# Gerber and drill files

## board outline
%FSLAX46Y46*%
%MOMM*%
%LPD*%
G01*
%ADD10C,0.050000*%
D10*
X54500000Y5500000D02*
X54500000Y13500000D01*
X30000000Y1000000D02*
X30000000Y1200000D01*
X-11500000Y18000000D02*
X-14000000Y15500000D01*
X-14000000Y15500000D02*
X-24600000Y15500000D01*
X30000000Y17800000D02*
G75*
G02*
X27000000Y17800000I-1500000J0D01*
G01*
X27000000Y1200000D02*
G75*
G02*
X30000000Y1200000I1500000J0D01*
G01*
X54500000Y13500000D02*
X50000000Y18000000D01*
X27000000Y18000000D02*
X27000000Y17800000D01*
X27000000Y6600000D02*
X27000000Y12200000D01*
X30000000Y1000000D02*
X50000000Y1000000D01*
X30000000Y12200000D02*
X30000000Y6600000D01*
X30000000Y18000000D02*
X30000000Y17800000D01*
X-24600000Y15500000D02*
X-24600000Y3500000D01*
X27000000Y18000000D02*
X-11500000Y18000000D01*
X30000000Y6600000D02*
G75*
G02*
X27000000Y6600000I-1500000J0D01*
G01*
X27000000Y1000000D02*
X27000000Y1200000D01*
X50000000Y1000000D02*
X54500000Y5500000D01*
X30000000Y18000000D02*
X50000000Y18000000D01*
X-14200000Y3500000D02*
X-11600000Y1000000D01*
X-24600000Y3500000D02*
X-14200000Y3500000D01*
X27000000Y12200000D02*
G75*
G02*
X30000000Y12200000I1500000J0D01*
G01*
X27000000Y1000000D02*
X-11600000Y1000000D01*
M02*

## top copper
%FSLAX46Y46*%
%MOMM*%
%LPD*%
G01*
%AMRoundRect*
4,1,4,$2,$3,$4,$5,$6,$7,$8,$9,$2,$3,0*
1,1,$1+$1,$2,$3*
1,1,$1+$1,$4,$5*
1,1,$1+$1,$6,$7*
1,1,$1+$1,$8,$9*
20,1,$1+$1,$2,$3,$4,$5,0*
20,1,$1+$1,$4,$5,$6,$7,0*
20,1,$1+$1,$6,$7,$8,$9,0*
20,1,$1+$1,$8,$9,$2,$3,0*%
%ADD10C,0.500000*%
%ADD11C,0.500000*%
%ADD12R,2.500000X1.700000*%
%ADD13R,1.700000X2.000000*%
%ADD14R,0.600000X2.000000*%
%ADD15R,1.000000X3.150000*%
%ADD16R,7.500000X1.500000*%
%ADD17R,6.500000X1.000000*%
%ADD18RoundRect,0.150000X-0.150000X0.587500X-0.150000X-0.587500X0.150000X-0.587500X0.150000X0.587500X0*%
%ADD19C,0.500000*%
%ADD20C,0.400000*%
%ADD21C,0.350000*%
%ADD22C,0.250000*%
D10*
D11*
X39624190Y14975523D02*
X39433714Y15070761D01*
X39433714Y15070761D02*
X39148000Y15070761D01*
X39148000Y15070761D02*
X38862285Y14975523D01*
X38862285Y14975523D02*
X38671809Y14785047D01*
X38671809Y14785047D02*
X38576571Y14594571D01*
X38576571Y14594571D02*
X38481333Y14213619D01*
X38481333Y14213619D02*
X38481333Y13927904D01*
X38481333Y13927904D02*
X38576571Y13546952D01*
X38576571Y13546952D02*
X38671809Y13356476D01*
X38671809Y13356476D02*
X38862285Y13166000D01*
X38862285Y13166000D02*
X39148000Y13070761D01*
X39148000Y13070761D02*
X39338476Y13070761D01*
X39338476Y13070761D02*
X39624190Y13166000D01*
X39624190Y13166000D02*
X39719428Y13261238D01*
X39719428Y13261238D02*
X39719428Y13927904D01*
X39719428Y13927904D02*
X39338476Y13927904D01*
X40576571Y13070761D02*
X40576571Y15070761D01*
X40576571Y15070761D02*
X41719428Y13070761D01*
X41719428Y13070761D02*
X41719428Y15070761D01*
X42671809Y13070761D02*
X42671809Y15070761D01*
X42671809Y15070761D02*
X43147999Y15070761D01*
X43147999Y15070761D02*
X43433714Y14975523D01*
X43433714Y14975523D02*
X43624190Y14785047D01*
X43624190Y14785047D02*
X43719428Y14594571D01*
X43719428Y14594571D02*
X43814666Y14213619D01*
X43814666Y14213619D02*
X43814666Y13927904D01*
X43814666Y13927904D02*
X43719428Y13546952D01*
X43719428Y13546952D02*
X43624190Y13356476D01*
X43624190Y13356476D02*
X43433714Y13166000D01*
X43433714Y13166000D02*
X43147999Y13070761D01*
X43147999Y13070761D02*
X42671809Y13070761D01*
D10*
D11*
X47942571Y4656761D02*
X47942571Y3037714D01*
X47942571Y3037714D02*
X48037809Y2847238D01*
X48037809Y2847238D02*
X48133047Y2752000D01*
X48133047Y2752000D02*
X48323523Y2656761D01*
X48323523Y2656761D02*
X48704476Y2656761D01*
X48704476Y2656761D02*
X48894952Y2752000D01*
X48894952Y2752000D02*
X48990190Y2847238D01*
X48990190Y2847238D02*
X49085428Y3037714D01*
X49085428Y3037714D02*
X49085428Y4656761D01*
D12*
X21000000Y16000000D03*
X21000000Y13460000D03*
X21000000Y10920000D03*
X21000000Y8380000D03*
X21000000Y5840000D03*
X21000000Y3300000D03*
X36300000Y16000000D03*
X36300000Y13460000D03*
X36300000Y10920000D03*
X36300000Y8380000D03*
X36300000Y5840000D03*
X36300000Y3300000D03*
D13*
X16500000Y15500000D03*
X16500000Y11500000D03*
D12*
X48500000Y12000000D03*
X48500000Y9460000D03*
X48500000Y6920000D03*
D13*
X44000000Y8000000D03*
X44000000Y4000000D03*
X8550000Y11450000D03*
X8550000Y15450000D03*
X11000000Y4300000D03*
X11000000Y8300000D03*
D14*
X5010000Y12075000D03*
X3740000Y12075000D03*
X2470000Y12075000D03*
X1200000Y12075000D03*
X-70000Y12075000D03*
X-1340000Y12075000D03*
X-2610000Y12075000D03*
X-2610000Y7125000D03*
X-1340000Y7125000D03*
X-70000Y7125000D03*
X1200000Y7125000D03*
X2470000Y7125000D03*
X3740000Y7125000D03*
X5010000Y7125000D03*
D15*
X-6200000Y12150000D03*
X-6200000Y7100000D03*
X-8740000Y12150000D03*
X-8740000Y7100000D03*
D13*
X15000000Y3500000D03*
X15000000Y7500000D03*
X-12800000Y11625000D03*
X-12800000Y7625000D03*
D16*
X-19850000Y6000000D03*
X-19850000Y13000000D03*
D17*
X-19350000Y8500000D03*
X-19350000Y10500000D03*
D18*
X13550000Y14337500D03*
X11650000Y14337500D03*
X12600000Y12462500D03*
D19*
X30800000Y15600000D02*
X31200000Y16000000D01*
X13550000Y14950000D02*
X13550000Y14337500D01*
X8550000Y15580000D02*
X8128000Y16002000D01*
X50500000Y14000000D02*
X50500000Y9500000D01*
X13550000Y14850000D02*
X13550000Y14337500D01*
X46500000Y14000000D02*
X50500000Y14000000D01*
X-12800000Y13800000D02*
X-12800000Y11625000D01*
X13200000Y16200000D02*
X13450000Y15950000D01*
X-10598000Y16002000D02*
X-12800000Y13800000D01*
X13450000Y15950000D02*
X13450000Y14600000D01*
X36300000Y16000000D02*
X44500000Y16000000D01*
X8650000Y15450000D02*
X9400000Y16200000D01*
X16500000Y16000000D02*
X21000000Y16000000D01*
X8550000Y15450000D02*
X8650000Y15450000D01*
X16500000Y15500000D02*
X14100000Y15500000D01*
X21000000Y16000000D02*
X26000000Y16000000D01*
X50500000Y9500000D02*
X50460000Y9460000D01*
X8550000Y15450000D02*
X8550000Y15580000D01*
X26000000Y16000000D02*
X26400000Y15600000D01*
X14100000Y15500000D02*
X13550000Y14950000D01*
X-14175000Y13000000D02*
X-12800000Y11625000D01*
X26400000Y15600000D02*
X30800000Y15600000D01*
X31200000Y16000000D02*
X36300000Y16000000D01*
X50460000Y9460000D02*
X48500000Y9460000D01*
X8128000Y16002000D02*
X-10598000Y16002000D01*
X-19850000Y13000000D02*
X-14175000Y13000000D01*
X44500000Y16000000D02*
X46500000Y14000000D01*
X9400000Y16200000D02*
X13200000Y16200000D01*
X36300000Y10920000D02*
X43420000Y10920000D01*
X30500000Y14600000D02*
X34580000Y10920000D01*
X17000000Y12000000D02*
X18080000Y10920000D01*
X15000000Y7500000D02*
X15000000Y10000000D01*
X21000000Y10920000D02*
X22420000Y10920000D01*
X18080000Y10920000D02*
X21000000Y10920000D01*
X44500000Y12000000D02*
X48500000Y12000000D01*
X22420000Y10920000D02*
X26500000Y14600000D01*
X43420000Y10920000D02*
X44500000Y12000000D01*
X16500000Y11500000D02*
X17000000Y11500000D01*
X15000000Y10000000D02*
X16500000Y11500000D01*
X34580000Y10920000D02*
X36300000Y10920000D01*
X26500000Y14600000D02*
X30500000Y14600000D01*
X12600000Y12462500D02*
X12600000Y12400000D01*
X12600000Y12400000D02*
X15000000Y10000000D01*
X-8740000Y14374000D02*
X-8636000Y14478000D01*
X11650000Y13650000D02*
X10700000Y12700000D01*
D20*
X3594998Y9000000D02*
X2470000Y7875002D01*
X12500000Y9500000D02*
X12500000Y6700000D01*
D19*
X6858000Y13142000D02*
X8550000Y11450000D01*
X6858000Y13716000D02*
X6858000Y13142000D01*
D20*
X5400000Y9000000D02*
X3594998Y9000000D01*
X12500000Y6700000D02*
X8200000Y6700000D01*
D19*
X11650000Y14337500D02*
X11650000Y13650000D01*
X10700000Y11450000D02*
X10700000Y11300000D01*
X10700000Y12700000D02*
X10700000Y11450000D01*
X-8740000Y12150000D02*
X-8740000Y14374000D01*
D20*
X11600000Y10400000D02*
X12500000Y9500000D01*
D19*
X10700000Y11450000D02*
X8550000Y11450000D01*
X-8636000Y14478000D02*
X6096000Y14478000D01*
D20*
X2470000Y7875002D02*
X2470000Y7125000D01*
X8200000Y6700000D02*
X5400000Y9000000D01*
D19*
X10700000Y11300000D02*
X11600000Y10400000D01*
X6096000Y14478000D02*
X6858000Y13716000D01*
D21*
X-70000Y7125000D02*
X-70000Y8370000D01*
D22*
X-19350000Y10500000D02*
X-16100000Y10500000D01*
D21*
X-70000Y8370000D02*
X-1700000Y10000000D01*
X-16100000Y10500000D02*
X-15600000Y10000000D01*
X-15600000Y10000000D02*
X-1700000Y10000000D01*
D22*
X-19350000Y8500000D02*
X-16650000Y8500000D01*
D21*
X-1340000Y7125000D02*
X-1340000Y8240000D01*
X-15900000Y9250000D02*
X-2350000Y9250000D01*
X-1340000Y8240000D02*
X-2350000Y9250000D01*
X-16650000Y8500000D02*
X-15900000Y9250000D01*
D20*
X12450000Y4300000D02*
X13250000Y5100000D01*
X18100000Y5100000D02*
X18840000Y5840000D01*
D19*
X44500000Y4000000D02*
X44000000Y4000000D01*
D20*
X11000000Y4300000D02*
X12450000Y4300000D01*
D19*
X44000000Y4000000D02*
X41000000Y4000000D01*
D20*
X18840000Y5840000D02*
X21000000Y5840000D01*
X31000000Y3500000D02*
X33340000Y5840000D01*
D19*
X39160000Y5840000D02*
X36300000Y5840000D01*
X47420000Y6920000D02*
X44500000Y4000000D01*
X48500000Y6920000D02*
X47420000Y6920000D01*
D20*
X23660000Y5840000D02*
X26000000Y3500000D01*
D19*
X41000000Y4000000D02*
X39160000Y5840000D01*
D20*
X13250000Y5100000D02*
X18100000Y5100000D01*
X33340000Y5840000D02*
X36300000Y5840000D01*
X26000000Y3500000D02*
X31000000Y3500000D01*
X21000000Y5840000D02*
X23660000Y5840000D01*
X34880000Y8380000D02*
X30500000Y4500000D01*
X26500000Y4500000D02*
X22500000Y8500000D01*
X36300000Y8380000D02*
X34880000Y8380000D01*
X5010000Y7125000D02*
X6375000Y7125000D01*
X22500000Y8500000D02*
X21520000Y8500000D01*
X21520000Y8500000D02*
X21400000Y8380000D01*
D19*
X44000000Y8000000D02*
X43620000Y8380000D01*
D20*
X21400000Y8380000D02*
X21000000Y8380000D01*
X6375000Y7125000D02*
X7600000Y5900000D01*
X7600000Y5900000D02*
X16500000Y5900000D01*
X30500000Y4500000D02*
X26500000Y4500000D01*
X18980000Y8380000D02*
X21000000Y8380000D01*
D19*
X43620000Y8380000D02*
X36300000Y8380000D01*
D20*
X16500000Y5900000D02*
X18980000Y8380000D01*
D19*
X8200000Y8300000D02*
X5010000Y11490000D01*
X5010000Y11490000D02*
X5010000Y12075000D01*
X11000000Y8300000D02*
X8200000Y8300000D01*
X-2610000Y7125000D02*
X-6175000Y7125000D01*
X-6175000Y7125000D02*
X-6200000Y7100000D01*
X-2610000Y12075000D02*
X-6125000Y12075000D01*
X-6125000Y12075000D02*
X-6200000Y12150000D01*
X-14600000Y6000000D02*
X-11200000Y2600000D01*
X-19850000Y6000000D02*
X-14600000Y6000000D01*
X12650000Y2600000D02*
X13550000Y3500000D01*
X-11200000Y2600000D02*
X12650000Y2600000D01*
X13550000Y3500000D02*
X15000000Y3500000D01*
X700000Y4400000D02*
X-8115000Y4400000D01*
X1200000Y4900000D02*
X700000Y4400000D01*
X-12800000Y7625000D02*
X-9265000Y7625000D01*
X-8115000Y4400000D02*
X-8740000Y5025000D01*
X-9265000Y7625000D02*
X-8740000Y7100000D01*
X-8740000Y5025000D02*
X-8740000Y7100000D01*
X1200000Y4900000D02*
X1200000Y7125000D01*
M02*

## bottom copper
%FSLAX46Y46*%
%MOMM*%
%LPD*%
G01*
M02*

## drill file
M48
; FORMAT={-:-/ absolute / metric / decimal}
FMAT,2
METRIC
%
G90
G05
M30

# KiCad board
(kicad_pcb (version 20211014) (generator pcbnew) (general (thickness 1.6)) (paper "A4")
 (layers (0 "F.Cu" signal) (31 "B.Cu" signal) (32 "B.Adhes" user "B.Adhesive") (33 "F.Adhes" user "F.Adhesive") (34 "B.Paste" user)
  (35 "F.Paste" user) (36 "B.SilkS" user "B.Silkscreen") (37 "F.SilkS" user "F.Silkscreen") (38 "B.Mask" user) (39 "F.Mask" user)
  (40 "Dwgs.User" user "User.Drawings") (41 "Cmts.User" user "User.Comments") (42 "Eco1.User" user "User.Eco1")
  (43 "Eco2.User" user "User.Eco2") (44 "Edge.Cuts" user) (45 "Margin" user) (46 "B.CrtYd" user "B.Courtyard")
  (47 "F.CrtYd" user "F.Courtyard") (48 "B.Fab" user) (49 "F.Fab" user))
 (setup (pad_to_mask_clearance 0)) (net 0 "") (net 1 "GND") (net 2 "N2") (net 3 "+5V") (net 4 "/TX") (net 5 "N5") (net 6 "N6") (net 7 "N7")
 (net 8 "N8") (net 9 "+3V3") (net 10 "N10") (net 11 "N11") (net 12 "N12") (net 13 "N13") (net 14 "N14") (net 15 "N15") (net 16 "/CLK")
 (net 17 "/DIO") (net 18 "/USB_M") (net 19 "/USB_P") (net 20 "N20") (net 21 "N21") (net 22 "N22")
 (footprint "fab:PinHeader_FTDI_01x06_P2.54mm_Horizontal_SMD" (layer "F.Cu") (at 21 -16)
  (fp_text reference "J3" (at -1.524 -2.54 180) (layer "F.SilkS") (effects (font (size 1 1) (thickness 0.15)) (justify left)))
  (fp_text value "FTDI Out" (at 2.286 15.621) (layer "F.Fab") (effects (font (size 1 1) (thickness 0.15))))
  (pad "1" smd rect locked (at 0 0) (size 2.5 1.7) (layers "F.Cu" "F.Paste" "F.Mask") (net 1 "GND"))
  (pad "2" smd rect locked (at 0 2.54) (size 2.5 1.7) (layers "F.Cu" "F.Paste" "F.Mask") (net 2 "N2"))
  (pad "3" smd rect locked (at 0 5.08) (size 2.5 1.7) (layers "F.Cu" "F.Paste" "F.Mask") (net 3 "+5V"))
  (pad "4" smd rect locked (at 0 7.62) (size 2.5 1.7) (layers "F.Cu" "F.Paste" "F.Mask") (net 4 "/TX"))
  (pad "5" smd rect locked (at 0 10.16) (size 2.5 1.7) (layers "F.Cu" "F.Paste" "F.Mask") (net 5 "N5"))
  (pad "6" smd rect locked (at 0 12.7) (size 2.5 1.7) (layers "F.Cu" "F.Paste" "F.Mask") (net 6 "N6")))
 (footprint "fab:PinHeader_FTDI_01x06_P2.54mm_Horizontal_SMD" (layer "F.Cu") (at 36.3 -16)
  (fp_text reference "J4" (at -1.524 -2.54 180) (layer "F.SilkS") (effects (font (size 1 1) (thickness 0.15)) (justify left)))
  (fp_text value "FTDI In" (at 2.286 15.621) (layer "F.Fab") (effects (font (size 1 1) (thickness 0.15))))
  (pad "1" smd rect locked (at 0 0) (size 2.5 1.7) (layers "F.Cu" "F.Paste" "F.Mask") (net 1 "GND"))
  (pad "2" smd rect locked (at 0 2.54) (size 2.5 1.7) (layers "F.Cu" "F.Paste" "F.Mask") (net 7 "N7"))
  (pad "3" smd rect locked (at 0 5.08) (size 2.5 1.7) (layers "F.Cu" "F.Paste" "F.Mask") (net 3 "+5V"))
  (pad "4" smd rect locked (at 0 7.62) (size 2.5 1.7) (layers "F.Cu" "F.Paste" "F.Mask") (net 4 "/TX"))
  (pad "5" smd rect locked (at 0 10.16) (size 2.5 1.7) (layers "F.Cu" "F.Paste" "F.Mask") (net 5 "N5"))
  (pad "6" smd rect locked (at 0 12.7) (size 2.5 1.7) (layers "F.Cu" "F.Paste" "F.Mask") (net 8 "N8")))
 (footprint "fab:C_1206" (layer "F.Cu") (at 16.5 -13.5 -90)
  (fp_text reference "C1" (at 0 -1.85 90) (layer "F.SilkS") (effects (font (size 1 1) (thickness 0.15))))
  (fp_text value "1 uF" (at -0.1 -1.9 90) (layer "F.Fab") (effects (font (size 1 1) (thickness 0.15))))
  (pad "1" smd rect locked (at -2 0 270) (size 2 1.7) (layers "F.Cu" "F.Paste" "F.Mask") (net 1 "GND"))
  (pad "2" smd rect locked (at 2 0 270) (size 2 1.7) (layers "F.Cu" "F.Paste" "F.Mask") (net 3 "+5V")))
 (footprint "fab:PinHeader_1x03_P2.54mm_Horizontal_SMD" (layer "F.Cu") (at 48.5 -12)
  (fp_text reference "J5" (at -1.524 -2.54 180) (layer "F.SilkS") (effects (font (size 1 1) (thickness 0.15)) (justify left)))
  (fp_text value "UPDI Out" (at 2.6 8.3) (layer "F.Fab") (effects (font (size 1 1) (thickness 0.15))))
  (pad "1" smd rect locked (at 0 0) (size 2.5 1.7) (layers "F.Cu" "F.Paste" "F.Mask") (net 3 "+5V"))
  (pad "2" smd rect locked (at 0 2.54) (size 2.5 1.7) (layers "F.Cu" "F.Paste" "F.Mask") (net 1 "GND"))
  (pad "3" smd rect locked (at 0 5.08) (size 2.5 1.7) (layers "F.Cu" "F.Paste" "F.Mask") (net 5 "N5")))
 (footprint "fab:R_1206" (layer "F.Cu") (at 44 -6 -90)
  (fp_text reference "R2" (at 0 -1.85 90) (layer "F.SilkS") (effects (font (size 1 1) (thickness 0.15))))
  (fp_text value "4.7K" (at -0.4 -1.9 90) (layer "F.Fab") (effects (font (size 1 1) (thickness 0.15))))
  (pad "1" smd rect locked (at -2 0 270) (size 2 1.7) (layers "F.Cu" "F.Paste" "F.Mask") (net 4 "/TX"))
  (pad "2" smd rect locked (at 2 0 270) (size 2 1.7) (layers "F.Cu" "F.Paste" "F.Mask") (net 5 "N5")))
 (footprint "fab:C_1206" (layer "F.Cu") (at 8.55 -13.45 90)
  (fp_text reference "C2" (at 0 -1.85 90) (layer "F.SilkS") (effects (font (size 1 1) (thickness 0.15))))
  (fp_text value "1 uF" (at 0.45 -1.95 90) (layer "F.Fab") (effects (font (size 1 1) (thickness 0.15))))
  (pad "1" smd rect locked (at -2 0 90) (size 2 1.7) (layers "F.Cu" "F.Paste" "F.Mask") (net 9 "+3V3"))
  (pad "2" smd rect locked (at 2 0 90) (size 2 1.7) (layers "F.Cu" "F.Paste" "F.Mask") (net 1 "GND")))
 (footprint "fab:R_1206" (layer "F.Cu") (at 11 -6.3 90)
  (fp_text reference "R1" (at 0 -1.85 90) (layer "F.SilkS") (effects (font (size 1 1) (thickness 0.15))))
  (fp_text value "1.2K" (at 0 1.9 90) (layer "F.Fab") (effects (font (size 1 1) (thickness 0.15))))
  (pad "1" smd rect locked (at -2 0 90) (size 2 1.7) (layers "F.Cu" "F.Paste" "F.Mask") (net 5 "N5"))
  (pad "2" smd rect locked (at 2 0 90) (size 2 1.7) (layers "F.Cu" "F.Paste" "F.Mask") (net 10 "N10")))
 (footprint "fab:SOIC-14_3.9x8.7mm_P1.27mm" (layer "F.Cu") (at 1.2 -9.6 -90)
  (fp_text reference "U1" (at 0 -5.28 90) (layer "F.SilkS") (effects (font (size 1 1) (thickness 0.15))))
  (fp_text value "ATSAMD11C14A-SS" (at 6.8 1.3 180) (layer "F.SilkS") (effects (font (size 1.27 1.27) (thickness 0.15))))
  (pad "1" smd rect locked (at -2.475 -3.81 270) (size 2 0.6) (layers "F.Cu" "F.Paste" "F.Mask") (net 10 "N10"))
  (pad "2" smd rect locked (at -2.475 -2.54 270) (size 2 0.6) (layers "F.Cu" "F.Paste" "F.Mask") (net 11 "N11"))
  (pad "3" smd rect locked (at -2.475 -1.27 270) (size 2 0.6) (layers "F.Cu" "F.Paste" "F.Mask") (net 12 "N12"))
  (pad "4" smd rect locked (at -2.475 0 270) (size 2 0.6) (layers "F.Cu" "F.Paste" "F.Mask") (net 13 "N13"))
  (pad "5" smd rect locked (at -2.475 1.27 270) (size 2 0.6) (layers "F.Cu" "F.Paste" "F.Mask") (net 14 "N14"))
  (pad "6" smd rect locked (at -2.475 2.54 270) (size 2 0.6) (layers "F.Cu" "F.Paste" "F.Mask") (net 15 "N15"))
  (pad "7" smd rect locked (at -2.475 3.81 270) (size 2 0.6) (layers "F.Cu" "F.Paste" "F.Mask") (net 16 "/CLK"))
  (pad "8" smd rect locked (at 2.475 3.81 270) (size 2 0.6) (layers "F.Cu" "F.Paste" "F.Mask") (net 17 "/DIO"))
  (pad "9" smd rect locked (at 2.475 2.54 270) (size 2 0.6) (layers "F.Cu" "F.Paste" "F.Mask") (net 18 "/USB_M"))
  (pad "10" smd rect locked (at 2.475 1.27 270) (size 2 0.6) (layers "F.Cu" "F.Paste" "F.Mask") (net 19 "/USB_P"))
  (pad "11" smd rect locked (at 2.475 0 270) (size 2 0.6) (layers "F.Cu" "F.Paste" "F.Mask") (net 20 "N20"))
  (pad "12" smd rect locked (at 2.475 -1.27 270) (size 2 0.6) (layers "F.Cu" "F.Paste" "F.Mask") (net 9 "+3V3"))
  (pad "13" smd rect locked (at 2.475 -2.54 270) (size 2 0.6) (layers "F.Cu" "F.Paste" "F.Mask") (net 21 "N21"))
  (pad "14" smd rect locked (at 2.475 -3.81 270) (size 2 0.6) (layers "F.Cu" "F.Paste" "F.Mask") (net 4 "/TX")))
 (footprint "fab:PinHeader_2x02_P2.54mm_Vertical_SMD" (layer "F.Cu") (at -7.47 -9.625 -90)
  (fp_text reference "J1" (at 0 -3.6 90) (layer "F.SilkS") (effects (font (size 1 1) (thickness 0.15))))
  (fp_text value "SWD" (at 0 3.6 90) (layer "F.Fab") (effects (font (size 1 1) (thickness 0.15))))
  (pad "1" smd rect locked (at -2.525 -1.27 270) (size 3.15 1) (layers "F.Cu" "F.Paste" "F.Mask") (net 16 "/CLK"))
  (pad "2" smd rect locked (at 2.525 -1.27 270) (size 3.15 1) (layers "F.Cu" "F.Paste" "F.Mask") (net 17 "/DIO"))
  (pad "3" smd rect locked (at -2.525 1.27 270) (size 3.15 1) (layers "F.Cu" "F.Paste" "F.Mask") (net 9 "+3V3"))
  (pad "4" smd rect locked (at 2.525 1.27 270) (size 3.15 1) (layers "F.Cu" "F.Paste" "F.Mask") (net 20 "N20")))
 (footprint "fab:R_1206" (layer "F.Cu") (at 15 -5.5 90)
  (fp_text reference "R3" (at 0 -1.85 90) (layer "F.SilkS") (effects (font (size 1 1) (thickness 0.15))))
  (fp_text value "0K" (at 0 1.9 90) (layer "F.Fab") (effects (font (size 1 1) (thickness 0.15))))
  (pad "1" smd rect locked (at -2 0 90) (size 2 1.7) (layers "F.Cu" "F.Paste" "F.Mask") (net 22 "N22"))
  (pad "2" smd rect locked (at 2 0 90) (size 2 1.7) (layers "F.Cu" "F.Paste" "F.Mask") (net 3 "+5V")))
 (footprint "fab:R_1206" (layer "F.Cu") (at -12.8 -9.625 -90)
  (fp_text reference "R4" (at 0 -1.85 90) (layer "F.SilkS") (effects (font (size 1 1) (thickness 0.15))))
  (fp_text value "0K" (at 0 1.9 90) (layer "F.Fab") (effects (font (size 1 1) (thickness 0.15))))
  (pad "1" smd rect locked (at -2 0 270) (size 2 1.7) (layers "F.Cu" "F.Paste" "F.Mask") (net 1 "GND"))
  (pad "2" smd rect locked (at 2 0 270) (size 2 1.7) (layers "F.Cu" "F.Paste" "F.Mask") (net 20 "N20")))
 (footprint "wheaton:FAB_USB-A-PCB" (layer "F.Cu") (at -19.65 -9.5)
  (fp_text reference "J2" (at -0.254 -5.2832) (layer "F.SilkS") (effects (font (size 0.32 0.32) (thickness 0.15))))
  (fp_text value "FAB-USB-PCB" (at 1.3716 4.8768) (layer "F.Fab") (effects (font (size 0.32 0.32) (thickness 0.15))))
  (pad "5V" smd rect locked (at -0.2 3.5) (size 7.5 1.5) (layers "F.Cu" "F.Paste" "F.Mask") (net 22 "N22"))
  (pad "GND" smd rect locked (at -0.2 -3.5) (size 7.5 1.5) (layers "F.Cu" "F.Paste" "F.Mask") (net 1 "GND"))
  (pad "USB_M" smd rect locked (at 0.3 1) (size 6.5 1) (layers "F.Cu" "F.Paste" "F.Mask") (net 18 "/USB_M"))
  (pad "USB_P" smd rect locked (at 0.3 -1) (size 6.5 1) (layers "F.Cu" "F.Paste" "F.Mask") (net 19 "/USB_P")))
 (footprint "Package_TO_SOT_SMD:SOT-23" (layer "F.Cu") (at 12.6 -13.4 -90)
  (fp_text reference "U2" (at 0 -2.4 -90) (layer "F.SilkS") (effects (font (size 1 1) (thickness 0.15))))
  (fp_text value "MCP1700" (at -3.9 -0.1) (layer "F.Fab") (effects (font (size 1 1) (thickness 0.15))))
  (pad "1" smd roundrect (at -0.9375 -0.95 270) (size 1.475 0.6) (layers "F.Cu" "F.Paste" "F.Mask") (roundrect_rratio 0.25) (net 1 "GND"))
  (pad "2" smd roundrect (at -0.9375 0.95 270) (size 1.475 0.6) (layers "F.Cu" "F.Paste" "F.Mask") (roundrect_rratio 0.25) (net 9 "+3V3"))
  (pad "3" smd roundrect (at 0.9375 0 270) (size 1.475 0.6) (layers "F.Cu" "F.Paste" "F.Mask") (roundrect_rratio 0.25) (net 3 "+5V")))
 (gr_line (start 54.5 -5.5) (end 54.5 -13.5) (layer "Edge.Cuts") (width 0.05))
 (gr_line (start 30 -1) (end 30 -1.2) (layer "Edge.Cuts") (width 0.05))
 (gr_line (start -11.5 -18) (end -14 -15.5) (layer "Edge.Cuts") (width 0.05))
 (gr_line (start -14 -15.5) (end -24.6 -15.5) (layer "Edge.Cuts") (width 0.05))
 (gr_arc (start 30 -17.8) (mid 28.5 -16.3) (end 27 -17.8) (layer "Edge.Cuts") (width 0.05))
 (gr_arc (start 27 -1.2) (mid 28.5 -2.7) (end 30 -1.2) (layer "Edge.Cuts") (width 0.05))
 (gr_line (start 54.5 -13.5) (end 50 -18) (layer "Edge.Cuts") (width 0.05))
 (gr_line (start 27 -18) (end 27 -17.8) (layer "Edge.Cuts") (width 0.05))
 (gr_line (start 27 -6.6) (end 27 -12.2) (layer "Edge.Cuts") (width 0.05))
 (gr_line (start 30 -1) (end 50 -1) (layer "Edge.Cuts") (width 0.05))
 (gr_line (start 30 -12.2) (end 30 -6.6) (layer "Edge.Cuts") (width 0.05))
 (gr_line (start 30 -18) (end 30 -17.8) (layer "Edge.Cuts") (width 0.05))
 (gr_line (start -24.6 -15.5) (end -24.6 -3.5) (layer "Edge.Cuts") (width 0.05))
 (gr_line (start 27 -18) (end -11.5 -18) (layer "Edge.Cuts") (width 0.05))
 (gr_arc (start 30 -6.6) (mid 28.5 -5.1) (end 27 -6.6) (layer "Edge.Cuts") (width 0.05))
 (gr_line (start 27 -1) (end 27 -1.2) (layer "Edge.Cuts") (width 0.05))
 (gr_line (start 50 -1) (end 54.5 -5.5) (layer "Edge.Cuts") (width 0.05))
 (gr_line (start 30 -18) (end 50 -18) (layer "Edge.Cuts") (width 0.05))
 (gr_line (start -14.2 -3.5) (end -11.6 -1) (layer "Edge.Cuts") (width 0.05))
 (gr_line (start -24.6 -3.5) (end -14.2 -3.5) (layer "Edge.Cuts") (width 0.05))
 (gr_arc (start 27 -12.2) (mid 28.5 -13.7) (end 30 -12.2) (layer "Edge.Cuts") (width 0.05))
 (gr_line (start 27 -1) (end -11.6 -1) (layer "Edge.Cuts") (width 0.05))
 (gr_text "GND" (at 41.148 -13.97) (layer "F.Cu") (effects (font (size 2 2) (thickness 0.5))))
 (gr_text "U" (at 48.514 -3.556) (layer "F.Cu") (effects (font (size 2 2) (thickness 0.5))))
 (segment (start 30.8 -15.6) (end 31.2 -16) (width 0.5) (layer "F.Cu") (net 1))
 (segment (start 13.55 -14.95) (end 13.55 -14.3375) (width 0.5) (layer "F.Cu") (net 1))
 (segment (start 8.55 -15.58) (end 8.128 -16.002) (width 0.5) (layer "F.Cu") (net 1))
 (segment (start 50.5 -14) (end 50.5 -9.5) (width 0.5) (layer "F.Cu") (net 1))
 (segment (start 13.55 -14.85) (end 13.55 -14.3375) (width 0.5) (layer "F.Cu") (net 1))
 (segment (start 46.5 -14) (end 50.5 -14) (width 0.5) (layer "F.Cu") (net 1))
 (segment (start -12.8 -13.8) (end -12.8 -11.625) (width 0.5) (layer "F.Cu") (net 1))
 (segment (start 13.2 -16.2) (end 13.45 -15.95) (width 0.5) (layer "F.Cu") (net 1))
 (segment (start -10.598 -16.002) (end -12.8 -13.8) (width 0.5) (layer "F.Cu") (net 1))
 (segment (start 13.45 -15.95) (end 13.45 -14.6) (width 0.5) (layer "F.Cu") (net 1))
 (segment (start 36.3 -16) (end 44.5 -16) (width 0.5) (layer "F.Cu") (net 1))
 (segment (start 8.65 -15.45) (end 9.4 -16.2) (width 0.5) (layer "F.Cu") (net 1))
 (segment (start 16.5 -16) (end 21 -16) (width 0.5) (layer "F.Cu") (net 1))
 (segment (start 8.55 -15.45) (end 8.65 -15.45) (width 0.5) (layer "F.Cu") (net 1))
 (segment (start 16.5 -15.5) (end 14.1 -15.5) (width 0.5) (layer "F.Cu") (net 1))
 (segment (start 21 -16) (end 26 -16) (width 0.5) (layer "F.Cu") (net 1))
 (segment (start 50.5 -9.5) (end 50.46 -9.46) (width 0.5) (layer "F.Cu") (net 1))
 (segment (start 8.55 -15.45) (end 8.55 -15.58) (width 0.5) (layer "F.Cu") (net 1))
 (segment (start 26 -16) (end 26.4 -15.6) (width 0.5) (layer "F.Cu") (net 1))
 (segment (start 14.1 -15.5) (end 13.55 -14.95) (width 0.5) (layer "F.Cu") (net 1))
 (segment (start -14.175 -13) (end -12.8 -11.625) (width 0.5) (layer "F.Cu") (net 1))
 (segment (start 26.4 -15.6) (end 30.8 -15.6) (width 0.5) (layer "F.Cu") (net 1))
 (segment (start 31.2 -16) (end 36.3 -16) (width 0.5) (layer "F.Cu") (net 1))
 (segment (start 50.46 -9.46) (end 48.5 -9.46) (width 0.5) (layer "F.Cu") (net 1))
 (segment (start 8.128 -16.002) (end -10.598 -16.002) (width 0.5) (layer "F.Cu") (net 1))
 (segment (start -19.85 -13) (end -14.175 -13) (width 0.5) (layer "F.Cu") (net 1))
 (segment (start 44.5 -16) (end 46.5 -14) (width 0.5) (layer "F.Cu") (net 1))
 (segment (start 9.4 -16.2) (end 13.2 -16.2) (width 0.5) (layer "F.Cu") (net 1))
 (segment (start 36.3 -10.92) (end 43.42 -10.92) (width 0.5) (layer "F.Cu") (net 3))
 (segment (start 30.5 -14.6) (end 34.58 -10.92) (width 0.5) (layer "F.Cu") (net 3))
 (segment (start 17 -12) (end 18.08 -10.92) (width 0.5) (layer "F.Cu") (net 3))
 (segment (start 15 -7.5) (end 15 -10) (width 0.5) (layer "F.Cu") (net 3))
 (segment (start 21 -10.92) (end 22.42 -10.92) (width 0.5) (layer "F.Cu") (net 3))
 (segment (start 18.08 -10.92) (end 21 -10.92) (width 0.5) (layer "F.Cu") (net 3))
 (segment (start 44.5 -12) (end 48.5 -12) (width 0.5) (layer "F.Cu") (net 3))
 (segment (start 22.42 -10.92) (end 26.5 -14.6) (width 0.5) (layer "F.Cu") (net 3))
 (segment (start 43.42 -10.92) (end 44.5 -12) (width 0.5) (layer "F.Cu") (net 3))
 (segment (start 16.5 -11.5) (end 17 -11.5) (width 0.5) (layer "F.Cu") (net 3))
 (segment (start 15 -10) (end 16.5 -11.5) (width 0.5) (layer "F.Cu") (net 3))
 (segment (start 34.58 -10.92) (end 36.3 -10.92) (width 0.5) (layer "F.Cu") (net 3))
 (segment (start 26.5 -14.6) (end 30.5 -14.6) (width 0.5) (layer "F.Cu") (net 3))
 (segment (start 12.6 -12.4625) (end 12.6 -12.4) (width 0.5) (layer "F.Cu") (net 3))
 (segment (start 12.6 -12.4) (end 15 -10) (width 0.5) (layer "F.Cu") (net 3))
 (segment (start -8.74 -14.374) (end -8.636 -14.478) (width 0.5) (layer "F.Cu") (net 9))
 (segment (start 11.65 -13.65) (end 10.7 -12.7) (width 0.5) (layer "F.Cu") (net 9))
 (segment (start 3.594998 -9) (end 2.47 -7.875002) (width 0.4) (layer "F.Cu") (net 9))
 (segment (start 12.5 -9.5) (end 12.5 -6.7) (width 0.4) (layer "F.Cu") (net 9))
 (segment (start 6.858 -13.142) (end 8.55 -11.45) (width 0.5) (layer "F.Cu") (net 9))
 (segment (start 6.858 -13.716) (end 6.858 -13.142) (width 0.5) (layer "F.Cu") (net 9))
 (segment (start 5.4 -9) (end 3.594998 -9) (width 0.4) (layer "F.Cu") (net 9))
 (segment (start 12.5 -6.7) (end 8.2 -6.7) (width 0.4) (layer "F.Cu") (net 9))
 (segment (start 11.65 -14.3375) (end 11.65 -13.65) (width 0.5) (layer "F.Cu") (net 9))
 (segment (start 10.7 -11.45) (end 10.7 -11.3) (width 0.5) (layer "F.Cu") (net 9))
 (segment (start 10.7 -12.7) (end 10.7 -11.45) (width 0.5) (layer "F.Cu") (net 9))
 (segment (start -8.74 -12.15) (end -8.74 -14.374) (width 0.5) (layer "F.Cu") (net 9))
 (segment (start 11.6 -10.4) (end 12.5 -9.5) (width 0.4) (layer "F.Cu") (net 9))
 (segment (start 10.7 -11.45) (end 8.55 -11.45) (width 0.5) (layer "F.Cu") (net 9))
 (segment (start -8.636 -14.478) (end 6.096 -14.478) (width 0.5) (layer "F.Cu") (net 9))
 (segment (start 2.47 -7.875002) (end 2.47 -7.125) (width 0.4) (layer "F.Cu") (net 9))
 (segment (start 8.2 -6.7) (end 5.4 -9) (width 0.4) (layer "F.Cu") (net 9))
 (segment (start 10.7 -11.3) (end 11.6 -10.4) (width 0.5) (layer "F.Cu") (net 9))
 (segment (start 6.096 -14.478) (end 6.858 -13.716) (width 0.5) (layer "F.Cu") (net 9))
 (segment (start -0.07 -7.125) (end -0.07 -8.37) (width 0.35) (layer "F.Cu") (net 19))
 (segment (start -19.35 -10.5) (end -16.1 -10.5) (width 0.25) (layer "F.Cu") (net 19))
 (segment (start -0.07 -8.37) (end -1.7 -10) (width 0.35) (layer "F.Cu") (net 19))
 (segment (start -16.1 -10.5) (end -15.6 -10) (width 0.35) (layer "F.Cu") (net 19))
 (segment (start -15.6 -10) (end -1.7 -10) (width 0.35) (layer "F.Cu") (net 19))
 (segment (start -19.35 -8.5) (end -16.65 -8.5) (width 0.25) (layer "F.Cu") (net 18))
 (segment (start -1.34 -7.125) (end -1.34 -8.24) (width 0.35) (layer "F.Cu") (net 18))
 (segment (start -15.9 -9.25) (end -2.35 -9.25) (width 0.35) (layer "F.Cu") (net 18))
 (segment (start -1.34 -8.24) (end -2.35 -9.25) (width 0.35) (layer "F.Cu") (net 18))
 (segment (start -16.65 -8.5) (end -15.9 -9.25) (width 0.35) (layer "F.Cu") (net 18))
 (segment (start 12.45 -4.3) (end 13.25 -5.1) (width 0.4) (layer "F.Cu") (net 5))
 (segment (start 18.1 -5.1) (end 18.84 -5.84) (width 0.4) (layer "F.Cu") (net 5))
 (segment (start 44.5 -4) (end 44 -4) (width 0.5) (layer "F.Cu") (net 5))
 (segment (start 11 -4.3) (end 12.45 -4.3) (width 0.4) (layer "F.Cu") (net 5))
 (segment (start 44 -4) (end 41 -4) (width 0.5) (layer "F.Cu") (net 5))
 (segment (start 18.84 -5.84) (end 21 -5.84) (width 0.4) (layer "F.Cu") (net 5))
 (segment (start 31 -3.5) (end 33.34 -5.84) (width 0.4) (layer "F.Cu") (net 5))
 (segment (start 39.16 -5.84) (end 36.3 -5.84) (width 0.5) (layer "F.Cu") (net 5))
 (segment (start 47.42 -6.92) (end 44.5 -4) (width 0.5) (layer "F.Cu") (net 5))
 (segment (start 48.5 -6.92) (end 47.42 -6.92) (width 0.5) (layer "F.Cu") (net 5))
 (segment (start 23.66 -5.84) (end 26 -3.5) (width 0.4) (layer "F.Cu") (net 5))
 (segment (start 41 -4) (end 39.16 -5.84) (width 0.5) (layer "F.Cu") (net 5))
 (segment (start 13.25 -5.1) (end 18.1 -5.1) (width 0.4) (layer "F.Cu") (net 5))
 (segment (start 33.34 -5.84) (end 36.3 -5.84) (width 0.4) (layer "F.Cu") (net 5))
 (segment (start 26 -3.5) (end 31 -3.5) (width 0.4) (layer "F.Cu") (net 5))
 (segment (start 21 -5.84) (end 23.66 -5.84) (width 0.4) (layer "F.Cu") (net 5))
 (segment (start 34.88 -8.38) (end 30.5 -4.5) (width 0.4) (layer "F.Cu") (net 4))
 (segment (start 26.5 -4.5) (end 22.5 -8.5) (width 0.4) (layer "F.Cu") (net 4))
 (segment (start 36.3 -8.38) (end 34.88 -8.38) (width 0.4) (layer "F.Cu") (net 4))
 (segment (start 5.01 -7.125) (end 6.375 -7.125) (width 0.4) (layer "F.Cu") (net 4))
 (segment (start 22.5 -8.5) (end 21.52 -8.5) (width 0.4) (layer "F.Cu") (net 4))
 (segment (start 21.52 -8.5) (end 21.4 -8.38) (width 0.4) (layer "F.Cu") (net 4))
 (segment (start 44 -8) (end 43.62 -8.38) (width 0.5) (layer "F.Cu") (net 4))
 (segment (start 21.4 -8.38) (end 21 -8.38) (width 0.4) (layer "F.Cu") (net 4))
 (segment (start 6.375 -7.125) (end 7.6 -5.9) (width 0.4) (layer "F.Cu") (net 4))
 (segment (start 7.6 -5.9) (end 16.5 -5.9) (width 0.4) (layer "F.Cu") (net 4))
 (segment (start 30.5 -4.5) (end 26.5 -4.5) (width 0.4) (layer "F.Cu") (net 4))
 (segment (start 18.98 -8.38) (end 21 -8.38) (width 0.4) (layer "F.Cu") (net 4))
 (segment (start 43.62 -8.38) (end 36.3 -8.38) (width 0.5) (layer "F.Cu") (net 4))
 (segment (start 16.5 -5.9) (end 18.98 -8.38) (width 0.4) (layer "F.Cu") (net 4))
 (segment (start 8.2 -8.3) (end 5.01 -11.49) (width 0.5) (layer "F.Cu") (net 10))
 (segment (start 5.01 -11.49) (end 5.01 -12.075) (width 0.5) (layer "F.Cu") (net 10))
 (segment (start 11 -8.3) (end 8.2 -8.3) (width 0.5) (layer "F.Cu") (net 10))
 (segment (start -2.61 -7.125) (end -6.175 -7.125) (width 0.5) (layer "F.Cu") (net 17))
 (segment (start -6.175 -7.125) (end -6.2 -7.1) (width 0.5) (layer "F.Cu") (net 17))
 (segment (start -2.61 -12.075) (end -6.125 -12.075) (width 0.5) (layer "F.Cu") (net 16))
 (segment (start -6.125 -12.075) (end -6.2 -12.15) (width 0.5) (layer "F.Cu") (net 16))
 (segment (start -14.6 -6) (end -11.2 -2.6) (width 0.5) (layer "F.Cu") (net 22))
 (segment (start -19.85 -6) (end -14.6 -6) (width 0.5) (layer "F.Cu") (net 22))
 (segment (start 12.65 -2.6) (end 13.55 -3.5) (width 0.5) (layer "F.Cu") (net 22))
 (segment (start -11.2 -2.6) (end 12.65 -2.6) (width 0.5) (layer "F.Cu") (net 22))
 (segment (start 13.55 -3.5) (end 15 -3.5) (width 0.5) (layer "F.Cu") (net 22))
 (segment (start 0.7 -4.4) (end -8.115 -4.4) (width 0.5) (layer "F.Cu") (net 20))
 (segment (start 1.2 -4.9) (end 0.7 -4.4) (width 0.5) (layer "F.Cu") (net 20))
 (segment (start -12.8 -7.625) (end -9.265 -7.625) (width 0.5) (layer "F.Cu") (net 20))
 (segment (start -8.115 -4.4) (end -8.74 -5.025) (width 0.5) (layer "F.Cu") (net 20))
 (segment (start -9.265 -7.625) (end -8.74 -7.1) (width 0.5) (layer "F.Cu") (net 20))
 (segment (start -8.74 -5.025) (end -8.74 -7.1) (width 0.5) (layer "F.Cu") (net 20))
 (segment (start 1.2 -4.9) (end 1.2 -7.125) (width 0.5) (layer "F.Cu") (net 20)))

